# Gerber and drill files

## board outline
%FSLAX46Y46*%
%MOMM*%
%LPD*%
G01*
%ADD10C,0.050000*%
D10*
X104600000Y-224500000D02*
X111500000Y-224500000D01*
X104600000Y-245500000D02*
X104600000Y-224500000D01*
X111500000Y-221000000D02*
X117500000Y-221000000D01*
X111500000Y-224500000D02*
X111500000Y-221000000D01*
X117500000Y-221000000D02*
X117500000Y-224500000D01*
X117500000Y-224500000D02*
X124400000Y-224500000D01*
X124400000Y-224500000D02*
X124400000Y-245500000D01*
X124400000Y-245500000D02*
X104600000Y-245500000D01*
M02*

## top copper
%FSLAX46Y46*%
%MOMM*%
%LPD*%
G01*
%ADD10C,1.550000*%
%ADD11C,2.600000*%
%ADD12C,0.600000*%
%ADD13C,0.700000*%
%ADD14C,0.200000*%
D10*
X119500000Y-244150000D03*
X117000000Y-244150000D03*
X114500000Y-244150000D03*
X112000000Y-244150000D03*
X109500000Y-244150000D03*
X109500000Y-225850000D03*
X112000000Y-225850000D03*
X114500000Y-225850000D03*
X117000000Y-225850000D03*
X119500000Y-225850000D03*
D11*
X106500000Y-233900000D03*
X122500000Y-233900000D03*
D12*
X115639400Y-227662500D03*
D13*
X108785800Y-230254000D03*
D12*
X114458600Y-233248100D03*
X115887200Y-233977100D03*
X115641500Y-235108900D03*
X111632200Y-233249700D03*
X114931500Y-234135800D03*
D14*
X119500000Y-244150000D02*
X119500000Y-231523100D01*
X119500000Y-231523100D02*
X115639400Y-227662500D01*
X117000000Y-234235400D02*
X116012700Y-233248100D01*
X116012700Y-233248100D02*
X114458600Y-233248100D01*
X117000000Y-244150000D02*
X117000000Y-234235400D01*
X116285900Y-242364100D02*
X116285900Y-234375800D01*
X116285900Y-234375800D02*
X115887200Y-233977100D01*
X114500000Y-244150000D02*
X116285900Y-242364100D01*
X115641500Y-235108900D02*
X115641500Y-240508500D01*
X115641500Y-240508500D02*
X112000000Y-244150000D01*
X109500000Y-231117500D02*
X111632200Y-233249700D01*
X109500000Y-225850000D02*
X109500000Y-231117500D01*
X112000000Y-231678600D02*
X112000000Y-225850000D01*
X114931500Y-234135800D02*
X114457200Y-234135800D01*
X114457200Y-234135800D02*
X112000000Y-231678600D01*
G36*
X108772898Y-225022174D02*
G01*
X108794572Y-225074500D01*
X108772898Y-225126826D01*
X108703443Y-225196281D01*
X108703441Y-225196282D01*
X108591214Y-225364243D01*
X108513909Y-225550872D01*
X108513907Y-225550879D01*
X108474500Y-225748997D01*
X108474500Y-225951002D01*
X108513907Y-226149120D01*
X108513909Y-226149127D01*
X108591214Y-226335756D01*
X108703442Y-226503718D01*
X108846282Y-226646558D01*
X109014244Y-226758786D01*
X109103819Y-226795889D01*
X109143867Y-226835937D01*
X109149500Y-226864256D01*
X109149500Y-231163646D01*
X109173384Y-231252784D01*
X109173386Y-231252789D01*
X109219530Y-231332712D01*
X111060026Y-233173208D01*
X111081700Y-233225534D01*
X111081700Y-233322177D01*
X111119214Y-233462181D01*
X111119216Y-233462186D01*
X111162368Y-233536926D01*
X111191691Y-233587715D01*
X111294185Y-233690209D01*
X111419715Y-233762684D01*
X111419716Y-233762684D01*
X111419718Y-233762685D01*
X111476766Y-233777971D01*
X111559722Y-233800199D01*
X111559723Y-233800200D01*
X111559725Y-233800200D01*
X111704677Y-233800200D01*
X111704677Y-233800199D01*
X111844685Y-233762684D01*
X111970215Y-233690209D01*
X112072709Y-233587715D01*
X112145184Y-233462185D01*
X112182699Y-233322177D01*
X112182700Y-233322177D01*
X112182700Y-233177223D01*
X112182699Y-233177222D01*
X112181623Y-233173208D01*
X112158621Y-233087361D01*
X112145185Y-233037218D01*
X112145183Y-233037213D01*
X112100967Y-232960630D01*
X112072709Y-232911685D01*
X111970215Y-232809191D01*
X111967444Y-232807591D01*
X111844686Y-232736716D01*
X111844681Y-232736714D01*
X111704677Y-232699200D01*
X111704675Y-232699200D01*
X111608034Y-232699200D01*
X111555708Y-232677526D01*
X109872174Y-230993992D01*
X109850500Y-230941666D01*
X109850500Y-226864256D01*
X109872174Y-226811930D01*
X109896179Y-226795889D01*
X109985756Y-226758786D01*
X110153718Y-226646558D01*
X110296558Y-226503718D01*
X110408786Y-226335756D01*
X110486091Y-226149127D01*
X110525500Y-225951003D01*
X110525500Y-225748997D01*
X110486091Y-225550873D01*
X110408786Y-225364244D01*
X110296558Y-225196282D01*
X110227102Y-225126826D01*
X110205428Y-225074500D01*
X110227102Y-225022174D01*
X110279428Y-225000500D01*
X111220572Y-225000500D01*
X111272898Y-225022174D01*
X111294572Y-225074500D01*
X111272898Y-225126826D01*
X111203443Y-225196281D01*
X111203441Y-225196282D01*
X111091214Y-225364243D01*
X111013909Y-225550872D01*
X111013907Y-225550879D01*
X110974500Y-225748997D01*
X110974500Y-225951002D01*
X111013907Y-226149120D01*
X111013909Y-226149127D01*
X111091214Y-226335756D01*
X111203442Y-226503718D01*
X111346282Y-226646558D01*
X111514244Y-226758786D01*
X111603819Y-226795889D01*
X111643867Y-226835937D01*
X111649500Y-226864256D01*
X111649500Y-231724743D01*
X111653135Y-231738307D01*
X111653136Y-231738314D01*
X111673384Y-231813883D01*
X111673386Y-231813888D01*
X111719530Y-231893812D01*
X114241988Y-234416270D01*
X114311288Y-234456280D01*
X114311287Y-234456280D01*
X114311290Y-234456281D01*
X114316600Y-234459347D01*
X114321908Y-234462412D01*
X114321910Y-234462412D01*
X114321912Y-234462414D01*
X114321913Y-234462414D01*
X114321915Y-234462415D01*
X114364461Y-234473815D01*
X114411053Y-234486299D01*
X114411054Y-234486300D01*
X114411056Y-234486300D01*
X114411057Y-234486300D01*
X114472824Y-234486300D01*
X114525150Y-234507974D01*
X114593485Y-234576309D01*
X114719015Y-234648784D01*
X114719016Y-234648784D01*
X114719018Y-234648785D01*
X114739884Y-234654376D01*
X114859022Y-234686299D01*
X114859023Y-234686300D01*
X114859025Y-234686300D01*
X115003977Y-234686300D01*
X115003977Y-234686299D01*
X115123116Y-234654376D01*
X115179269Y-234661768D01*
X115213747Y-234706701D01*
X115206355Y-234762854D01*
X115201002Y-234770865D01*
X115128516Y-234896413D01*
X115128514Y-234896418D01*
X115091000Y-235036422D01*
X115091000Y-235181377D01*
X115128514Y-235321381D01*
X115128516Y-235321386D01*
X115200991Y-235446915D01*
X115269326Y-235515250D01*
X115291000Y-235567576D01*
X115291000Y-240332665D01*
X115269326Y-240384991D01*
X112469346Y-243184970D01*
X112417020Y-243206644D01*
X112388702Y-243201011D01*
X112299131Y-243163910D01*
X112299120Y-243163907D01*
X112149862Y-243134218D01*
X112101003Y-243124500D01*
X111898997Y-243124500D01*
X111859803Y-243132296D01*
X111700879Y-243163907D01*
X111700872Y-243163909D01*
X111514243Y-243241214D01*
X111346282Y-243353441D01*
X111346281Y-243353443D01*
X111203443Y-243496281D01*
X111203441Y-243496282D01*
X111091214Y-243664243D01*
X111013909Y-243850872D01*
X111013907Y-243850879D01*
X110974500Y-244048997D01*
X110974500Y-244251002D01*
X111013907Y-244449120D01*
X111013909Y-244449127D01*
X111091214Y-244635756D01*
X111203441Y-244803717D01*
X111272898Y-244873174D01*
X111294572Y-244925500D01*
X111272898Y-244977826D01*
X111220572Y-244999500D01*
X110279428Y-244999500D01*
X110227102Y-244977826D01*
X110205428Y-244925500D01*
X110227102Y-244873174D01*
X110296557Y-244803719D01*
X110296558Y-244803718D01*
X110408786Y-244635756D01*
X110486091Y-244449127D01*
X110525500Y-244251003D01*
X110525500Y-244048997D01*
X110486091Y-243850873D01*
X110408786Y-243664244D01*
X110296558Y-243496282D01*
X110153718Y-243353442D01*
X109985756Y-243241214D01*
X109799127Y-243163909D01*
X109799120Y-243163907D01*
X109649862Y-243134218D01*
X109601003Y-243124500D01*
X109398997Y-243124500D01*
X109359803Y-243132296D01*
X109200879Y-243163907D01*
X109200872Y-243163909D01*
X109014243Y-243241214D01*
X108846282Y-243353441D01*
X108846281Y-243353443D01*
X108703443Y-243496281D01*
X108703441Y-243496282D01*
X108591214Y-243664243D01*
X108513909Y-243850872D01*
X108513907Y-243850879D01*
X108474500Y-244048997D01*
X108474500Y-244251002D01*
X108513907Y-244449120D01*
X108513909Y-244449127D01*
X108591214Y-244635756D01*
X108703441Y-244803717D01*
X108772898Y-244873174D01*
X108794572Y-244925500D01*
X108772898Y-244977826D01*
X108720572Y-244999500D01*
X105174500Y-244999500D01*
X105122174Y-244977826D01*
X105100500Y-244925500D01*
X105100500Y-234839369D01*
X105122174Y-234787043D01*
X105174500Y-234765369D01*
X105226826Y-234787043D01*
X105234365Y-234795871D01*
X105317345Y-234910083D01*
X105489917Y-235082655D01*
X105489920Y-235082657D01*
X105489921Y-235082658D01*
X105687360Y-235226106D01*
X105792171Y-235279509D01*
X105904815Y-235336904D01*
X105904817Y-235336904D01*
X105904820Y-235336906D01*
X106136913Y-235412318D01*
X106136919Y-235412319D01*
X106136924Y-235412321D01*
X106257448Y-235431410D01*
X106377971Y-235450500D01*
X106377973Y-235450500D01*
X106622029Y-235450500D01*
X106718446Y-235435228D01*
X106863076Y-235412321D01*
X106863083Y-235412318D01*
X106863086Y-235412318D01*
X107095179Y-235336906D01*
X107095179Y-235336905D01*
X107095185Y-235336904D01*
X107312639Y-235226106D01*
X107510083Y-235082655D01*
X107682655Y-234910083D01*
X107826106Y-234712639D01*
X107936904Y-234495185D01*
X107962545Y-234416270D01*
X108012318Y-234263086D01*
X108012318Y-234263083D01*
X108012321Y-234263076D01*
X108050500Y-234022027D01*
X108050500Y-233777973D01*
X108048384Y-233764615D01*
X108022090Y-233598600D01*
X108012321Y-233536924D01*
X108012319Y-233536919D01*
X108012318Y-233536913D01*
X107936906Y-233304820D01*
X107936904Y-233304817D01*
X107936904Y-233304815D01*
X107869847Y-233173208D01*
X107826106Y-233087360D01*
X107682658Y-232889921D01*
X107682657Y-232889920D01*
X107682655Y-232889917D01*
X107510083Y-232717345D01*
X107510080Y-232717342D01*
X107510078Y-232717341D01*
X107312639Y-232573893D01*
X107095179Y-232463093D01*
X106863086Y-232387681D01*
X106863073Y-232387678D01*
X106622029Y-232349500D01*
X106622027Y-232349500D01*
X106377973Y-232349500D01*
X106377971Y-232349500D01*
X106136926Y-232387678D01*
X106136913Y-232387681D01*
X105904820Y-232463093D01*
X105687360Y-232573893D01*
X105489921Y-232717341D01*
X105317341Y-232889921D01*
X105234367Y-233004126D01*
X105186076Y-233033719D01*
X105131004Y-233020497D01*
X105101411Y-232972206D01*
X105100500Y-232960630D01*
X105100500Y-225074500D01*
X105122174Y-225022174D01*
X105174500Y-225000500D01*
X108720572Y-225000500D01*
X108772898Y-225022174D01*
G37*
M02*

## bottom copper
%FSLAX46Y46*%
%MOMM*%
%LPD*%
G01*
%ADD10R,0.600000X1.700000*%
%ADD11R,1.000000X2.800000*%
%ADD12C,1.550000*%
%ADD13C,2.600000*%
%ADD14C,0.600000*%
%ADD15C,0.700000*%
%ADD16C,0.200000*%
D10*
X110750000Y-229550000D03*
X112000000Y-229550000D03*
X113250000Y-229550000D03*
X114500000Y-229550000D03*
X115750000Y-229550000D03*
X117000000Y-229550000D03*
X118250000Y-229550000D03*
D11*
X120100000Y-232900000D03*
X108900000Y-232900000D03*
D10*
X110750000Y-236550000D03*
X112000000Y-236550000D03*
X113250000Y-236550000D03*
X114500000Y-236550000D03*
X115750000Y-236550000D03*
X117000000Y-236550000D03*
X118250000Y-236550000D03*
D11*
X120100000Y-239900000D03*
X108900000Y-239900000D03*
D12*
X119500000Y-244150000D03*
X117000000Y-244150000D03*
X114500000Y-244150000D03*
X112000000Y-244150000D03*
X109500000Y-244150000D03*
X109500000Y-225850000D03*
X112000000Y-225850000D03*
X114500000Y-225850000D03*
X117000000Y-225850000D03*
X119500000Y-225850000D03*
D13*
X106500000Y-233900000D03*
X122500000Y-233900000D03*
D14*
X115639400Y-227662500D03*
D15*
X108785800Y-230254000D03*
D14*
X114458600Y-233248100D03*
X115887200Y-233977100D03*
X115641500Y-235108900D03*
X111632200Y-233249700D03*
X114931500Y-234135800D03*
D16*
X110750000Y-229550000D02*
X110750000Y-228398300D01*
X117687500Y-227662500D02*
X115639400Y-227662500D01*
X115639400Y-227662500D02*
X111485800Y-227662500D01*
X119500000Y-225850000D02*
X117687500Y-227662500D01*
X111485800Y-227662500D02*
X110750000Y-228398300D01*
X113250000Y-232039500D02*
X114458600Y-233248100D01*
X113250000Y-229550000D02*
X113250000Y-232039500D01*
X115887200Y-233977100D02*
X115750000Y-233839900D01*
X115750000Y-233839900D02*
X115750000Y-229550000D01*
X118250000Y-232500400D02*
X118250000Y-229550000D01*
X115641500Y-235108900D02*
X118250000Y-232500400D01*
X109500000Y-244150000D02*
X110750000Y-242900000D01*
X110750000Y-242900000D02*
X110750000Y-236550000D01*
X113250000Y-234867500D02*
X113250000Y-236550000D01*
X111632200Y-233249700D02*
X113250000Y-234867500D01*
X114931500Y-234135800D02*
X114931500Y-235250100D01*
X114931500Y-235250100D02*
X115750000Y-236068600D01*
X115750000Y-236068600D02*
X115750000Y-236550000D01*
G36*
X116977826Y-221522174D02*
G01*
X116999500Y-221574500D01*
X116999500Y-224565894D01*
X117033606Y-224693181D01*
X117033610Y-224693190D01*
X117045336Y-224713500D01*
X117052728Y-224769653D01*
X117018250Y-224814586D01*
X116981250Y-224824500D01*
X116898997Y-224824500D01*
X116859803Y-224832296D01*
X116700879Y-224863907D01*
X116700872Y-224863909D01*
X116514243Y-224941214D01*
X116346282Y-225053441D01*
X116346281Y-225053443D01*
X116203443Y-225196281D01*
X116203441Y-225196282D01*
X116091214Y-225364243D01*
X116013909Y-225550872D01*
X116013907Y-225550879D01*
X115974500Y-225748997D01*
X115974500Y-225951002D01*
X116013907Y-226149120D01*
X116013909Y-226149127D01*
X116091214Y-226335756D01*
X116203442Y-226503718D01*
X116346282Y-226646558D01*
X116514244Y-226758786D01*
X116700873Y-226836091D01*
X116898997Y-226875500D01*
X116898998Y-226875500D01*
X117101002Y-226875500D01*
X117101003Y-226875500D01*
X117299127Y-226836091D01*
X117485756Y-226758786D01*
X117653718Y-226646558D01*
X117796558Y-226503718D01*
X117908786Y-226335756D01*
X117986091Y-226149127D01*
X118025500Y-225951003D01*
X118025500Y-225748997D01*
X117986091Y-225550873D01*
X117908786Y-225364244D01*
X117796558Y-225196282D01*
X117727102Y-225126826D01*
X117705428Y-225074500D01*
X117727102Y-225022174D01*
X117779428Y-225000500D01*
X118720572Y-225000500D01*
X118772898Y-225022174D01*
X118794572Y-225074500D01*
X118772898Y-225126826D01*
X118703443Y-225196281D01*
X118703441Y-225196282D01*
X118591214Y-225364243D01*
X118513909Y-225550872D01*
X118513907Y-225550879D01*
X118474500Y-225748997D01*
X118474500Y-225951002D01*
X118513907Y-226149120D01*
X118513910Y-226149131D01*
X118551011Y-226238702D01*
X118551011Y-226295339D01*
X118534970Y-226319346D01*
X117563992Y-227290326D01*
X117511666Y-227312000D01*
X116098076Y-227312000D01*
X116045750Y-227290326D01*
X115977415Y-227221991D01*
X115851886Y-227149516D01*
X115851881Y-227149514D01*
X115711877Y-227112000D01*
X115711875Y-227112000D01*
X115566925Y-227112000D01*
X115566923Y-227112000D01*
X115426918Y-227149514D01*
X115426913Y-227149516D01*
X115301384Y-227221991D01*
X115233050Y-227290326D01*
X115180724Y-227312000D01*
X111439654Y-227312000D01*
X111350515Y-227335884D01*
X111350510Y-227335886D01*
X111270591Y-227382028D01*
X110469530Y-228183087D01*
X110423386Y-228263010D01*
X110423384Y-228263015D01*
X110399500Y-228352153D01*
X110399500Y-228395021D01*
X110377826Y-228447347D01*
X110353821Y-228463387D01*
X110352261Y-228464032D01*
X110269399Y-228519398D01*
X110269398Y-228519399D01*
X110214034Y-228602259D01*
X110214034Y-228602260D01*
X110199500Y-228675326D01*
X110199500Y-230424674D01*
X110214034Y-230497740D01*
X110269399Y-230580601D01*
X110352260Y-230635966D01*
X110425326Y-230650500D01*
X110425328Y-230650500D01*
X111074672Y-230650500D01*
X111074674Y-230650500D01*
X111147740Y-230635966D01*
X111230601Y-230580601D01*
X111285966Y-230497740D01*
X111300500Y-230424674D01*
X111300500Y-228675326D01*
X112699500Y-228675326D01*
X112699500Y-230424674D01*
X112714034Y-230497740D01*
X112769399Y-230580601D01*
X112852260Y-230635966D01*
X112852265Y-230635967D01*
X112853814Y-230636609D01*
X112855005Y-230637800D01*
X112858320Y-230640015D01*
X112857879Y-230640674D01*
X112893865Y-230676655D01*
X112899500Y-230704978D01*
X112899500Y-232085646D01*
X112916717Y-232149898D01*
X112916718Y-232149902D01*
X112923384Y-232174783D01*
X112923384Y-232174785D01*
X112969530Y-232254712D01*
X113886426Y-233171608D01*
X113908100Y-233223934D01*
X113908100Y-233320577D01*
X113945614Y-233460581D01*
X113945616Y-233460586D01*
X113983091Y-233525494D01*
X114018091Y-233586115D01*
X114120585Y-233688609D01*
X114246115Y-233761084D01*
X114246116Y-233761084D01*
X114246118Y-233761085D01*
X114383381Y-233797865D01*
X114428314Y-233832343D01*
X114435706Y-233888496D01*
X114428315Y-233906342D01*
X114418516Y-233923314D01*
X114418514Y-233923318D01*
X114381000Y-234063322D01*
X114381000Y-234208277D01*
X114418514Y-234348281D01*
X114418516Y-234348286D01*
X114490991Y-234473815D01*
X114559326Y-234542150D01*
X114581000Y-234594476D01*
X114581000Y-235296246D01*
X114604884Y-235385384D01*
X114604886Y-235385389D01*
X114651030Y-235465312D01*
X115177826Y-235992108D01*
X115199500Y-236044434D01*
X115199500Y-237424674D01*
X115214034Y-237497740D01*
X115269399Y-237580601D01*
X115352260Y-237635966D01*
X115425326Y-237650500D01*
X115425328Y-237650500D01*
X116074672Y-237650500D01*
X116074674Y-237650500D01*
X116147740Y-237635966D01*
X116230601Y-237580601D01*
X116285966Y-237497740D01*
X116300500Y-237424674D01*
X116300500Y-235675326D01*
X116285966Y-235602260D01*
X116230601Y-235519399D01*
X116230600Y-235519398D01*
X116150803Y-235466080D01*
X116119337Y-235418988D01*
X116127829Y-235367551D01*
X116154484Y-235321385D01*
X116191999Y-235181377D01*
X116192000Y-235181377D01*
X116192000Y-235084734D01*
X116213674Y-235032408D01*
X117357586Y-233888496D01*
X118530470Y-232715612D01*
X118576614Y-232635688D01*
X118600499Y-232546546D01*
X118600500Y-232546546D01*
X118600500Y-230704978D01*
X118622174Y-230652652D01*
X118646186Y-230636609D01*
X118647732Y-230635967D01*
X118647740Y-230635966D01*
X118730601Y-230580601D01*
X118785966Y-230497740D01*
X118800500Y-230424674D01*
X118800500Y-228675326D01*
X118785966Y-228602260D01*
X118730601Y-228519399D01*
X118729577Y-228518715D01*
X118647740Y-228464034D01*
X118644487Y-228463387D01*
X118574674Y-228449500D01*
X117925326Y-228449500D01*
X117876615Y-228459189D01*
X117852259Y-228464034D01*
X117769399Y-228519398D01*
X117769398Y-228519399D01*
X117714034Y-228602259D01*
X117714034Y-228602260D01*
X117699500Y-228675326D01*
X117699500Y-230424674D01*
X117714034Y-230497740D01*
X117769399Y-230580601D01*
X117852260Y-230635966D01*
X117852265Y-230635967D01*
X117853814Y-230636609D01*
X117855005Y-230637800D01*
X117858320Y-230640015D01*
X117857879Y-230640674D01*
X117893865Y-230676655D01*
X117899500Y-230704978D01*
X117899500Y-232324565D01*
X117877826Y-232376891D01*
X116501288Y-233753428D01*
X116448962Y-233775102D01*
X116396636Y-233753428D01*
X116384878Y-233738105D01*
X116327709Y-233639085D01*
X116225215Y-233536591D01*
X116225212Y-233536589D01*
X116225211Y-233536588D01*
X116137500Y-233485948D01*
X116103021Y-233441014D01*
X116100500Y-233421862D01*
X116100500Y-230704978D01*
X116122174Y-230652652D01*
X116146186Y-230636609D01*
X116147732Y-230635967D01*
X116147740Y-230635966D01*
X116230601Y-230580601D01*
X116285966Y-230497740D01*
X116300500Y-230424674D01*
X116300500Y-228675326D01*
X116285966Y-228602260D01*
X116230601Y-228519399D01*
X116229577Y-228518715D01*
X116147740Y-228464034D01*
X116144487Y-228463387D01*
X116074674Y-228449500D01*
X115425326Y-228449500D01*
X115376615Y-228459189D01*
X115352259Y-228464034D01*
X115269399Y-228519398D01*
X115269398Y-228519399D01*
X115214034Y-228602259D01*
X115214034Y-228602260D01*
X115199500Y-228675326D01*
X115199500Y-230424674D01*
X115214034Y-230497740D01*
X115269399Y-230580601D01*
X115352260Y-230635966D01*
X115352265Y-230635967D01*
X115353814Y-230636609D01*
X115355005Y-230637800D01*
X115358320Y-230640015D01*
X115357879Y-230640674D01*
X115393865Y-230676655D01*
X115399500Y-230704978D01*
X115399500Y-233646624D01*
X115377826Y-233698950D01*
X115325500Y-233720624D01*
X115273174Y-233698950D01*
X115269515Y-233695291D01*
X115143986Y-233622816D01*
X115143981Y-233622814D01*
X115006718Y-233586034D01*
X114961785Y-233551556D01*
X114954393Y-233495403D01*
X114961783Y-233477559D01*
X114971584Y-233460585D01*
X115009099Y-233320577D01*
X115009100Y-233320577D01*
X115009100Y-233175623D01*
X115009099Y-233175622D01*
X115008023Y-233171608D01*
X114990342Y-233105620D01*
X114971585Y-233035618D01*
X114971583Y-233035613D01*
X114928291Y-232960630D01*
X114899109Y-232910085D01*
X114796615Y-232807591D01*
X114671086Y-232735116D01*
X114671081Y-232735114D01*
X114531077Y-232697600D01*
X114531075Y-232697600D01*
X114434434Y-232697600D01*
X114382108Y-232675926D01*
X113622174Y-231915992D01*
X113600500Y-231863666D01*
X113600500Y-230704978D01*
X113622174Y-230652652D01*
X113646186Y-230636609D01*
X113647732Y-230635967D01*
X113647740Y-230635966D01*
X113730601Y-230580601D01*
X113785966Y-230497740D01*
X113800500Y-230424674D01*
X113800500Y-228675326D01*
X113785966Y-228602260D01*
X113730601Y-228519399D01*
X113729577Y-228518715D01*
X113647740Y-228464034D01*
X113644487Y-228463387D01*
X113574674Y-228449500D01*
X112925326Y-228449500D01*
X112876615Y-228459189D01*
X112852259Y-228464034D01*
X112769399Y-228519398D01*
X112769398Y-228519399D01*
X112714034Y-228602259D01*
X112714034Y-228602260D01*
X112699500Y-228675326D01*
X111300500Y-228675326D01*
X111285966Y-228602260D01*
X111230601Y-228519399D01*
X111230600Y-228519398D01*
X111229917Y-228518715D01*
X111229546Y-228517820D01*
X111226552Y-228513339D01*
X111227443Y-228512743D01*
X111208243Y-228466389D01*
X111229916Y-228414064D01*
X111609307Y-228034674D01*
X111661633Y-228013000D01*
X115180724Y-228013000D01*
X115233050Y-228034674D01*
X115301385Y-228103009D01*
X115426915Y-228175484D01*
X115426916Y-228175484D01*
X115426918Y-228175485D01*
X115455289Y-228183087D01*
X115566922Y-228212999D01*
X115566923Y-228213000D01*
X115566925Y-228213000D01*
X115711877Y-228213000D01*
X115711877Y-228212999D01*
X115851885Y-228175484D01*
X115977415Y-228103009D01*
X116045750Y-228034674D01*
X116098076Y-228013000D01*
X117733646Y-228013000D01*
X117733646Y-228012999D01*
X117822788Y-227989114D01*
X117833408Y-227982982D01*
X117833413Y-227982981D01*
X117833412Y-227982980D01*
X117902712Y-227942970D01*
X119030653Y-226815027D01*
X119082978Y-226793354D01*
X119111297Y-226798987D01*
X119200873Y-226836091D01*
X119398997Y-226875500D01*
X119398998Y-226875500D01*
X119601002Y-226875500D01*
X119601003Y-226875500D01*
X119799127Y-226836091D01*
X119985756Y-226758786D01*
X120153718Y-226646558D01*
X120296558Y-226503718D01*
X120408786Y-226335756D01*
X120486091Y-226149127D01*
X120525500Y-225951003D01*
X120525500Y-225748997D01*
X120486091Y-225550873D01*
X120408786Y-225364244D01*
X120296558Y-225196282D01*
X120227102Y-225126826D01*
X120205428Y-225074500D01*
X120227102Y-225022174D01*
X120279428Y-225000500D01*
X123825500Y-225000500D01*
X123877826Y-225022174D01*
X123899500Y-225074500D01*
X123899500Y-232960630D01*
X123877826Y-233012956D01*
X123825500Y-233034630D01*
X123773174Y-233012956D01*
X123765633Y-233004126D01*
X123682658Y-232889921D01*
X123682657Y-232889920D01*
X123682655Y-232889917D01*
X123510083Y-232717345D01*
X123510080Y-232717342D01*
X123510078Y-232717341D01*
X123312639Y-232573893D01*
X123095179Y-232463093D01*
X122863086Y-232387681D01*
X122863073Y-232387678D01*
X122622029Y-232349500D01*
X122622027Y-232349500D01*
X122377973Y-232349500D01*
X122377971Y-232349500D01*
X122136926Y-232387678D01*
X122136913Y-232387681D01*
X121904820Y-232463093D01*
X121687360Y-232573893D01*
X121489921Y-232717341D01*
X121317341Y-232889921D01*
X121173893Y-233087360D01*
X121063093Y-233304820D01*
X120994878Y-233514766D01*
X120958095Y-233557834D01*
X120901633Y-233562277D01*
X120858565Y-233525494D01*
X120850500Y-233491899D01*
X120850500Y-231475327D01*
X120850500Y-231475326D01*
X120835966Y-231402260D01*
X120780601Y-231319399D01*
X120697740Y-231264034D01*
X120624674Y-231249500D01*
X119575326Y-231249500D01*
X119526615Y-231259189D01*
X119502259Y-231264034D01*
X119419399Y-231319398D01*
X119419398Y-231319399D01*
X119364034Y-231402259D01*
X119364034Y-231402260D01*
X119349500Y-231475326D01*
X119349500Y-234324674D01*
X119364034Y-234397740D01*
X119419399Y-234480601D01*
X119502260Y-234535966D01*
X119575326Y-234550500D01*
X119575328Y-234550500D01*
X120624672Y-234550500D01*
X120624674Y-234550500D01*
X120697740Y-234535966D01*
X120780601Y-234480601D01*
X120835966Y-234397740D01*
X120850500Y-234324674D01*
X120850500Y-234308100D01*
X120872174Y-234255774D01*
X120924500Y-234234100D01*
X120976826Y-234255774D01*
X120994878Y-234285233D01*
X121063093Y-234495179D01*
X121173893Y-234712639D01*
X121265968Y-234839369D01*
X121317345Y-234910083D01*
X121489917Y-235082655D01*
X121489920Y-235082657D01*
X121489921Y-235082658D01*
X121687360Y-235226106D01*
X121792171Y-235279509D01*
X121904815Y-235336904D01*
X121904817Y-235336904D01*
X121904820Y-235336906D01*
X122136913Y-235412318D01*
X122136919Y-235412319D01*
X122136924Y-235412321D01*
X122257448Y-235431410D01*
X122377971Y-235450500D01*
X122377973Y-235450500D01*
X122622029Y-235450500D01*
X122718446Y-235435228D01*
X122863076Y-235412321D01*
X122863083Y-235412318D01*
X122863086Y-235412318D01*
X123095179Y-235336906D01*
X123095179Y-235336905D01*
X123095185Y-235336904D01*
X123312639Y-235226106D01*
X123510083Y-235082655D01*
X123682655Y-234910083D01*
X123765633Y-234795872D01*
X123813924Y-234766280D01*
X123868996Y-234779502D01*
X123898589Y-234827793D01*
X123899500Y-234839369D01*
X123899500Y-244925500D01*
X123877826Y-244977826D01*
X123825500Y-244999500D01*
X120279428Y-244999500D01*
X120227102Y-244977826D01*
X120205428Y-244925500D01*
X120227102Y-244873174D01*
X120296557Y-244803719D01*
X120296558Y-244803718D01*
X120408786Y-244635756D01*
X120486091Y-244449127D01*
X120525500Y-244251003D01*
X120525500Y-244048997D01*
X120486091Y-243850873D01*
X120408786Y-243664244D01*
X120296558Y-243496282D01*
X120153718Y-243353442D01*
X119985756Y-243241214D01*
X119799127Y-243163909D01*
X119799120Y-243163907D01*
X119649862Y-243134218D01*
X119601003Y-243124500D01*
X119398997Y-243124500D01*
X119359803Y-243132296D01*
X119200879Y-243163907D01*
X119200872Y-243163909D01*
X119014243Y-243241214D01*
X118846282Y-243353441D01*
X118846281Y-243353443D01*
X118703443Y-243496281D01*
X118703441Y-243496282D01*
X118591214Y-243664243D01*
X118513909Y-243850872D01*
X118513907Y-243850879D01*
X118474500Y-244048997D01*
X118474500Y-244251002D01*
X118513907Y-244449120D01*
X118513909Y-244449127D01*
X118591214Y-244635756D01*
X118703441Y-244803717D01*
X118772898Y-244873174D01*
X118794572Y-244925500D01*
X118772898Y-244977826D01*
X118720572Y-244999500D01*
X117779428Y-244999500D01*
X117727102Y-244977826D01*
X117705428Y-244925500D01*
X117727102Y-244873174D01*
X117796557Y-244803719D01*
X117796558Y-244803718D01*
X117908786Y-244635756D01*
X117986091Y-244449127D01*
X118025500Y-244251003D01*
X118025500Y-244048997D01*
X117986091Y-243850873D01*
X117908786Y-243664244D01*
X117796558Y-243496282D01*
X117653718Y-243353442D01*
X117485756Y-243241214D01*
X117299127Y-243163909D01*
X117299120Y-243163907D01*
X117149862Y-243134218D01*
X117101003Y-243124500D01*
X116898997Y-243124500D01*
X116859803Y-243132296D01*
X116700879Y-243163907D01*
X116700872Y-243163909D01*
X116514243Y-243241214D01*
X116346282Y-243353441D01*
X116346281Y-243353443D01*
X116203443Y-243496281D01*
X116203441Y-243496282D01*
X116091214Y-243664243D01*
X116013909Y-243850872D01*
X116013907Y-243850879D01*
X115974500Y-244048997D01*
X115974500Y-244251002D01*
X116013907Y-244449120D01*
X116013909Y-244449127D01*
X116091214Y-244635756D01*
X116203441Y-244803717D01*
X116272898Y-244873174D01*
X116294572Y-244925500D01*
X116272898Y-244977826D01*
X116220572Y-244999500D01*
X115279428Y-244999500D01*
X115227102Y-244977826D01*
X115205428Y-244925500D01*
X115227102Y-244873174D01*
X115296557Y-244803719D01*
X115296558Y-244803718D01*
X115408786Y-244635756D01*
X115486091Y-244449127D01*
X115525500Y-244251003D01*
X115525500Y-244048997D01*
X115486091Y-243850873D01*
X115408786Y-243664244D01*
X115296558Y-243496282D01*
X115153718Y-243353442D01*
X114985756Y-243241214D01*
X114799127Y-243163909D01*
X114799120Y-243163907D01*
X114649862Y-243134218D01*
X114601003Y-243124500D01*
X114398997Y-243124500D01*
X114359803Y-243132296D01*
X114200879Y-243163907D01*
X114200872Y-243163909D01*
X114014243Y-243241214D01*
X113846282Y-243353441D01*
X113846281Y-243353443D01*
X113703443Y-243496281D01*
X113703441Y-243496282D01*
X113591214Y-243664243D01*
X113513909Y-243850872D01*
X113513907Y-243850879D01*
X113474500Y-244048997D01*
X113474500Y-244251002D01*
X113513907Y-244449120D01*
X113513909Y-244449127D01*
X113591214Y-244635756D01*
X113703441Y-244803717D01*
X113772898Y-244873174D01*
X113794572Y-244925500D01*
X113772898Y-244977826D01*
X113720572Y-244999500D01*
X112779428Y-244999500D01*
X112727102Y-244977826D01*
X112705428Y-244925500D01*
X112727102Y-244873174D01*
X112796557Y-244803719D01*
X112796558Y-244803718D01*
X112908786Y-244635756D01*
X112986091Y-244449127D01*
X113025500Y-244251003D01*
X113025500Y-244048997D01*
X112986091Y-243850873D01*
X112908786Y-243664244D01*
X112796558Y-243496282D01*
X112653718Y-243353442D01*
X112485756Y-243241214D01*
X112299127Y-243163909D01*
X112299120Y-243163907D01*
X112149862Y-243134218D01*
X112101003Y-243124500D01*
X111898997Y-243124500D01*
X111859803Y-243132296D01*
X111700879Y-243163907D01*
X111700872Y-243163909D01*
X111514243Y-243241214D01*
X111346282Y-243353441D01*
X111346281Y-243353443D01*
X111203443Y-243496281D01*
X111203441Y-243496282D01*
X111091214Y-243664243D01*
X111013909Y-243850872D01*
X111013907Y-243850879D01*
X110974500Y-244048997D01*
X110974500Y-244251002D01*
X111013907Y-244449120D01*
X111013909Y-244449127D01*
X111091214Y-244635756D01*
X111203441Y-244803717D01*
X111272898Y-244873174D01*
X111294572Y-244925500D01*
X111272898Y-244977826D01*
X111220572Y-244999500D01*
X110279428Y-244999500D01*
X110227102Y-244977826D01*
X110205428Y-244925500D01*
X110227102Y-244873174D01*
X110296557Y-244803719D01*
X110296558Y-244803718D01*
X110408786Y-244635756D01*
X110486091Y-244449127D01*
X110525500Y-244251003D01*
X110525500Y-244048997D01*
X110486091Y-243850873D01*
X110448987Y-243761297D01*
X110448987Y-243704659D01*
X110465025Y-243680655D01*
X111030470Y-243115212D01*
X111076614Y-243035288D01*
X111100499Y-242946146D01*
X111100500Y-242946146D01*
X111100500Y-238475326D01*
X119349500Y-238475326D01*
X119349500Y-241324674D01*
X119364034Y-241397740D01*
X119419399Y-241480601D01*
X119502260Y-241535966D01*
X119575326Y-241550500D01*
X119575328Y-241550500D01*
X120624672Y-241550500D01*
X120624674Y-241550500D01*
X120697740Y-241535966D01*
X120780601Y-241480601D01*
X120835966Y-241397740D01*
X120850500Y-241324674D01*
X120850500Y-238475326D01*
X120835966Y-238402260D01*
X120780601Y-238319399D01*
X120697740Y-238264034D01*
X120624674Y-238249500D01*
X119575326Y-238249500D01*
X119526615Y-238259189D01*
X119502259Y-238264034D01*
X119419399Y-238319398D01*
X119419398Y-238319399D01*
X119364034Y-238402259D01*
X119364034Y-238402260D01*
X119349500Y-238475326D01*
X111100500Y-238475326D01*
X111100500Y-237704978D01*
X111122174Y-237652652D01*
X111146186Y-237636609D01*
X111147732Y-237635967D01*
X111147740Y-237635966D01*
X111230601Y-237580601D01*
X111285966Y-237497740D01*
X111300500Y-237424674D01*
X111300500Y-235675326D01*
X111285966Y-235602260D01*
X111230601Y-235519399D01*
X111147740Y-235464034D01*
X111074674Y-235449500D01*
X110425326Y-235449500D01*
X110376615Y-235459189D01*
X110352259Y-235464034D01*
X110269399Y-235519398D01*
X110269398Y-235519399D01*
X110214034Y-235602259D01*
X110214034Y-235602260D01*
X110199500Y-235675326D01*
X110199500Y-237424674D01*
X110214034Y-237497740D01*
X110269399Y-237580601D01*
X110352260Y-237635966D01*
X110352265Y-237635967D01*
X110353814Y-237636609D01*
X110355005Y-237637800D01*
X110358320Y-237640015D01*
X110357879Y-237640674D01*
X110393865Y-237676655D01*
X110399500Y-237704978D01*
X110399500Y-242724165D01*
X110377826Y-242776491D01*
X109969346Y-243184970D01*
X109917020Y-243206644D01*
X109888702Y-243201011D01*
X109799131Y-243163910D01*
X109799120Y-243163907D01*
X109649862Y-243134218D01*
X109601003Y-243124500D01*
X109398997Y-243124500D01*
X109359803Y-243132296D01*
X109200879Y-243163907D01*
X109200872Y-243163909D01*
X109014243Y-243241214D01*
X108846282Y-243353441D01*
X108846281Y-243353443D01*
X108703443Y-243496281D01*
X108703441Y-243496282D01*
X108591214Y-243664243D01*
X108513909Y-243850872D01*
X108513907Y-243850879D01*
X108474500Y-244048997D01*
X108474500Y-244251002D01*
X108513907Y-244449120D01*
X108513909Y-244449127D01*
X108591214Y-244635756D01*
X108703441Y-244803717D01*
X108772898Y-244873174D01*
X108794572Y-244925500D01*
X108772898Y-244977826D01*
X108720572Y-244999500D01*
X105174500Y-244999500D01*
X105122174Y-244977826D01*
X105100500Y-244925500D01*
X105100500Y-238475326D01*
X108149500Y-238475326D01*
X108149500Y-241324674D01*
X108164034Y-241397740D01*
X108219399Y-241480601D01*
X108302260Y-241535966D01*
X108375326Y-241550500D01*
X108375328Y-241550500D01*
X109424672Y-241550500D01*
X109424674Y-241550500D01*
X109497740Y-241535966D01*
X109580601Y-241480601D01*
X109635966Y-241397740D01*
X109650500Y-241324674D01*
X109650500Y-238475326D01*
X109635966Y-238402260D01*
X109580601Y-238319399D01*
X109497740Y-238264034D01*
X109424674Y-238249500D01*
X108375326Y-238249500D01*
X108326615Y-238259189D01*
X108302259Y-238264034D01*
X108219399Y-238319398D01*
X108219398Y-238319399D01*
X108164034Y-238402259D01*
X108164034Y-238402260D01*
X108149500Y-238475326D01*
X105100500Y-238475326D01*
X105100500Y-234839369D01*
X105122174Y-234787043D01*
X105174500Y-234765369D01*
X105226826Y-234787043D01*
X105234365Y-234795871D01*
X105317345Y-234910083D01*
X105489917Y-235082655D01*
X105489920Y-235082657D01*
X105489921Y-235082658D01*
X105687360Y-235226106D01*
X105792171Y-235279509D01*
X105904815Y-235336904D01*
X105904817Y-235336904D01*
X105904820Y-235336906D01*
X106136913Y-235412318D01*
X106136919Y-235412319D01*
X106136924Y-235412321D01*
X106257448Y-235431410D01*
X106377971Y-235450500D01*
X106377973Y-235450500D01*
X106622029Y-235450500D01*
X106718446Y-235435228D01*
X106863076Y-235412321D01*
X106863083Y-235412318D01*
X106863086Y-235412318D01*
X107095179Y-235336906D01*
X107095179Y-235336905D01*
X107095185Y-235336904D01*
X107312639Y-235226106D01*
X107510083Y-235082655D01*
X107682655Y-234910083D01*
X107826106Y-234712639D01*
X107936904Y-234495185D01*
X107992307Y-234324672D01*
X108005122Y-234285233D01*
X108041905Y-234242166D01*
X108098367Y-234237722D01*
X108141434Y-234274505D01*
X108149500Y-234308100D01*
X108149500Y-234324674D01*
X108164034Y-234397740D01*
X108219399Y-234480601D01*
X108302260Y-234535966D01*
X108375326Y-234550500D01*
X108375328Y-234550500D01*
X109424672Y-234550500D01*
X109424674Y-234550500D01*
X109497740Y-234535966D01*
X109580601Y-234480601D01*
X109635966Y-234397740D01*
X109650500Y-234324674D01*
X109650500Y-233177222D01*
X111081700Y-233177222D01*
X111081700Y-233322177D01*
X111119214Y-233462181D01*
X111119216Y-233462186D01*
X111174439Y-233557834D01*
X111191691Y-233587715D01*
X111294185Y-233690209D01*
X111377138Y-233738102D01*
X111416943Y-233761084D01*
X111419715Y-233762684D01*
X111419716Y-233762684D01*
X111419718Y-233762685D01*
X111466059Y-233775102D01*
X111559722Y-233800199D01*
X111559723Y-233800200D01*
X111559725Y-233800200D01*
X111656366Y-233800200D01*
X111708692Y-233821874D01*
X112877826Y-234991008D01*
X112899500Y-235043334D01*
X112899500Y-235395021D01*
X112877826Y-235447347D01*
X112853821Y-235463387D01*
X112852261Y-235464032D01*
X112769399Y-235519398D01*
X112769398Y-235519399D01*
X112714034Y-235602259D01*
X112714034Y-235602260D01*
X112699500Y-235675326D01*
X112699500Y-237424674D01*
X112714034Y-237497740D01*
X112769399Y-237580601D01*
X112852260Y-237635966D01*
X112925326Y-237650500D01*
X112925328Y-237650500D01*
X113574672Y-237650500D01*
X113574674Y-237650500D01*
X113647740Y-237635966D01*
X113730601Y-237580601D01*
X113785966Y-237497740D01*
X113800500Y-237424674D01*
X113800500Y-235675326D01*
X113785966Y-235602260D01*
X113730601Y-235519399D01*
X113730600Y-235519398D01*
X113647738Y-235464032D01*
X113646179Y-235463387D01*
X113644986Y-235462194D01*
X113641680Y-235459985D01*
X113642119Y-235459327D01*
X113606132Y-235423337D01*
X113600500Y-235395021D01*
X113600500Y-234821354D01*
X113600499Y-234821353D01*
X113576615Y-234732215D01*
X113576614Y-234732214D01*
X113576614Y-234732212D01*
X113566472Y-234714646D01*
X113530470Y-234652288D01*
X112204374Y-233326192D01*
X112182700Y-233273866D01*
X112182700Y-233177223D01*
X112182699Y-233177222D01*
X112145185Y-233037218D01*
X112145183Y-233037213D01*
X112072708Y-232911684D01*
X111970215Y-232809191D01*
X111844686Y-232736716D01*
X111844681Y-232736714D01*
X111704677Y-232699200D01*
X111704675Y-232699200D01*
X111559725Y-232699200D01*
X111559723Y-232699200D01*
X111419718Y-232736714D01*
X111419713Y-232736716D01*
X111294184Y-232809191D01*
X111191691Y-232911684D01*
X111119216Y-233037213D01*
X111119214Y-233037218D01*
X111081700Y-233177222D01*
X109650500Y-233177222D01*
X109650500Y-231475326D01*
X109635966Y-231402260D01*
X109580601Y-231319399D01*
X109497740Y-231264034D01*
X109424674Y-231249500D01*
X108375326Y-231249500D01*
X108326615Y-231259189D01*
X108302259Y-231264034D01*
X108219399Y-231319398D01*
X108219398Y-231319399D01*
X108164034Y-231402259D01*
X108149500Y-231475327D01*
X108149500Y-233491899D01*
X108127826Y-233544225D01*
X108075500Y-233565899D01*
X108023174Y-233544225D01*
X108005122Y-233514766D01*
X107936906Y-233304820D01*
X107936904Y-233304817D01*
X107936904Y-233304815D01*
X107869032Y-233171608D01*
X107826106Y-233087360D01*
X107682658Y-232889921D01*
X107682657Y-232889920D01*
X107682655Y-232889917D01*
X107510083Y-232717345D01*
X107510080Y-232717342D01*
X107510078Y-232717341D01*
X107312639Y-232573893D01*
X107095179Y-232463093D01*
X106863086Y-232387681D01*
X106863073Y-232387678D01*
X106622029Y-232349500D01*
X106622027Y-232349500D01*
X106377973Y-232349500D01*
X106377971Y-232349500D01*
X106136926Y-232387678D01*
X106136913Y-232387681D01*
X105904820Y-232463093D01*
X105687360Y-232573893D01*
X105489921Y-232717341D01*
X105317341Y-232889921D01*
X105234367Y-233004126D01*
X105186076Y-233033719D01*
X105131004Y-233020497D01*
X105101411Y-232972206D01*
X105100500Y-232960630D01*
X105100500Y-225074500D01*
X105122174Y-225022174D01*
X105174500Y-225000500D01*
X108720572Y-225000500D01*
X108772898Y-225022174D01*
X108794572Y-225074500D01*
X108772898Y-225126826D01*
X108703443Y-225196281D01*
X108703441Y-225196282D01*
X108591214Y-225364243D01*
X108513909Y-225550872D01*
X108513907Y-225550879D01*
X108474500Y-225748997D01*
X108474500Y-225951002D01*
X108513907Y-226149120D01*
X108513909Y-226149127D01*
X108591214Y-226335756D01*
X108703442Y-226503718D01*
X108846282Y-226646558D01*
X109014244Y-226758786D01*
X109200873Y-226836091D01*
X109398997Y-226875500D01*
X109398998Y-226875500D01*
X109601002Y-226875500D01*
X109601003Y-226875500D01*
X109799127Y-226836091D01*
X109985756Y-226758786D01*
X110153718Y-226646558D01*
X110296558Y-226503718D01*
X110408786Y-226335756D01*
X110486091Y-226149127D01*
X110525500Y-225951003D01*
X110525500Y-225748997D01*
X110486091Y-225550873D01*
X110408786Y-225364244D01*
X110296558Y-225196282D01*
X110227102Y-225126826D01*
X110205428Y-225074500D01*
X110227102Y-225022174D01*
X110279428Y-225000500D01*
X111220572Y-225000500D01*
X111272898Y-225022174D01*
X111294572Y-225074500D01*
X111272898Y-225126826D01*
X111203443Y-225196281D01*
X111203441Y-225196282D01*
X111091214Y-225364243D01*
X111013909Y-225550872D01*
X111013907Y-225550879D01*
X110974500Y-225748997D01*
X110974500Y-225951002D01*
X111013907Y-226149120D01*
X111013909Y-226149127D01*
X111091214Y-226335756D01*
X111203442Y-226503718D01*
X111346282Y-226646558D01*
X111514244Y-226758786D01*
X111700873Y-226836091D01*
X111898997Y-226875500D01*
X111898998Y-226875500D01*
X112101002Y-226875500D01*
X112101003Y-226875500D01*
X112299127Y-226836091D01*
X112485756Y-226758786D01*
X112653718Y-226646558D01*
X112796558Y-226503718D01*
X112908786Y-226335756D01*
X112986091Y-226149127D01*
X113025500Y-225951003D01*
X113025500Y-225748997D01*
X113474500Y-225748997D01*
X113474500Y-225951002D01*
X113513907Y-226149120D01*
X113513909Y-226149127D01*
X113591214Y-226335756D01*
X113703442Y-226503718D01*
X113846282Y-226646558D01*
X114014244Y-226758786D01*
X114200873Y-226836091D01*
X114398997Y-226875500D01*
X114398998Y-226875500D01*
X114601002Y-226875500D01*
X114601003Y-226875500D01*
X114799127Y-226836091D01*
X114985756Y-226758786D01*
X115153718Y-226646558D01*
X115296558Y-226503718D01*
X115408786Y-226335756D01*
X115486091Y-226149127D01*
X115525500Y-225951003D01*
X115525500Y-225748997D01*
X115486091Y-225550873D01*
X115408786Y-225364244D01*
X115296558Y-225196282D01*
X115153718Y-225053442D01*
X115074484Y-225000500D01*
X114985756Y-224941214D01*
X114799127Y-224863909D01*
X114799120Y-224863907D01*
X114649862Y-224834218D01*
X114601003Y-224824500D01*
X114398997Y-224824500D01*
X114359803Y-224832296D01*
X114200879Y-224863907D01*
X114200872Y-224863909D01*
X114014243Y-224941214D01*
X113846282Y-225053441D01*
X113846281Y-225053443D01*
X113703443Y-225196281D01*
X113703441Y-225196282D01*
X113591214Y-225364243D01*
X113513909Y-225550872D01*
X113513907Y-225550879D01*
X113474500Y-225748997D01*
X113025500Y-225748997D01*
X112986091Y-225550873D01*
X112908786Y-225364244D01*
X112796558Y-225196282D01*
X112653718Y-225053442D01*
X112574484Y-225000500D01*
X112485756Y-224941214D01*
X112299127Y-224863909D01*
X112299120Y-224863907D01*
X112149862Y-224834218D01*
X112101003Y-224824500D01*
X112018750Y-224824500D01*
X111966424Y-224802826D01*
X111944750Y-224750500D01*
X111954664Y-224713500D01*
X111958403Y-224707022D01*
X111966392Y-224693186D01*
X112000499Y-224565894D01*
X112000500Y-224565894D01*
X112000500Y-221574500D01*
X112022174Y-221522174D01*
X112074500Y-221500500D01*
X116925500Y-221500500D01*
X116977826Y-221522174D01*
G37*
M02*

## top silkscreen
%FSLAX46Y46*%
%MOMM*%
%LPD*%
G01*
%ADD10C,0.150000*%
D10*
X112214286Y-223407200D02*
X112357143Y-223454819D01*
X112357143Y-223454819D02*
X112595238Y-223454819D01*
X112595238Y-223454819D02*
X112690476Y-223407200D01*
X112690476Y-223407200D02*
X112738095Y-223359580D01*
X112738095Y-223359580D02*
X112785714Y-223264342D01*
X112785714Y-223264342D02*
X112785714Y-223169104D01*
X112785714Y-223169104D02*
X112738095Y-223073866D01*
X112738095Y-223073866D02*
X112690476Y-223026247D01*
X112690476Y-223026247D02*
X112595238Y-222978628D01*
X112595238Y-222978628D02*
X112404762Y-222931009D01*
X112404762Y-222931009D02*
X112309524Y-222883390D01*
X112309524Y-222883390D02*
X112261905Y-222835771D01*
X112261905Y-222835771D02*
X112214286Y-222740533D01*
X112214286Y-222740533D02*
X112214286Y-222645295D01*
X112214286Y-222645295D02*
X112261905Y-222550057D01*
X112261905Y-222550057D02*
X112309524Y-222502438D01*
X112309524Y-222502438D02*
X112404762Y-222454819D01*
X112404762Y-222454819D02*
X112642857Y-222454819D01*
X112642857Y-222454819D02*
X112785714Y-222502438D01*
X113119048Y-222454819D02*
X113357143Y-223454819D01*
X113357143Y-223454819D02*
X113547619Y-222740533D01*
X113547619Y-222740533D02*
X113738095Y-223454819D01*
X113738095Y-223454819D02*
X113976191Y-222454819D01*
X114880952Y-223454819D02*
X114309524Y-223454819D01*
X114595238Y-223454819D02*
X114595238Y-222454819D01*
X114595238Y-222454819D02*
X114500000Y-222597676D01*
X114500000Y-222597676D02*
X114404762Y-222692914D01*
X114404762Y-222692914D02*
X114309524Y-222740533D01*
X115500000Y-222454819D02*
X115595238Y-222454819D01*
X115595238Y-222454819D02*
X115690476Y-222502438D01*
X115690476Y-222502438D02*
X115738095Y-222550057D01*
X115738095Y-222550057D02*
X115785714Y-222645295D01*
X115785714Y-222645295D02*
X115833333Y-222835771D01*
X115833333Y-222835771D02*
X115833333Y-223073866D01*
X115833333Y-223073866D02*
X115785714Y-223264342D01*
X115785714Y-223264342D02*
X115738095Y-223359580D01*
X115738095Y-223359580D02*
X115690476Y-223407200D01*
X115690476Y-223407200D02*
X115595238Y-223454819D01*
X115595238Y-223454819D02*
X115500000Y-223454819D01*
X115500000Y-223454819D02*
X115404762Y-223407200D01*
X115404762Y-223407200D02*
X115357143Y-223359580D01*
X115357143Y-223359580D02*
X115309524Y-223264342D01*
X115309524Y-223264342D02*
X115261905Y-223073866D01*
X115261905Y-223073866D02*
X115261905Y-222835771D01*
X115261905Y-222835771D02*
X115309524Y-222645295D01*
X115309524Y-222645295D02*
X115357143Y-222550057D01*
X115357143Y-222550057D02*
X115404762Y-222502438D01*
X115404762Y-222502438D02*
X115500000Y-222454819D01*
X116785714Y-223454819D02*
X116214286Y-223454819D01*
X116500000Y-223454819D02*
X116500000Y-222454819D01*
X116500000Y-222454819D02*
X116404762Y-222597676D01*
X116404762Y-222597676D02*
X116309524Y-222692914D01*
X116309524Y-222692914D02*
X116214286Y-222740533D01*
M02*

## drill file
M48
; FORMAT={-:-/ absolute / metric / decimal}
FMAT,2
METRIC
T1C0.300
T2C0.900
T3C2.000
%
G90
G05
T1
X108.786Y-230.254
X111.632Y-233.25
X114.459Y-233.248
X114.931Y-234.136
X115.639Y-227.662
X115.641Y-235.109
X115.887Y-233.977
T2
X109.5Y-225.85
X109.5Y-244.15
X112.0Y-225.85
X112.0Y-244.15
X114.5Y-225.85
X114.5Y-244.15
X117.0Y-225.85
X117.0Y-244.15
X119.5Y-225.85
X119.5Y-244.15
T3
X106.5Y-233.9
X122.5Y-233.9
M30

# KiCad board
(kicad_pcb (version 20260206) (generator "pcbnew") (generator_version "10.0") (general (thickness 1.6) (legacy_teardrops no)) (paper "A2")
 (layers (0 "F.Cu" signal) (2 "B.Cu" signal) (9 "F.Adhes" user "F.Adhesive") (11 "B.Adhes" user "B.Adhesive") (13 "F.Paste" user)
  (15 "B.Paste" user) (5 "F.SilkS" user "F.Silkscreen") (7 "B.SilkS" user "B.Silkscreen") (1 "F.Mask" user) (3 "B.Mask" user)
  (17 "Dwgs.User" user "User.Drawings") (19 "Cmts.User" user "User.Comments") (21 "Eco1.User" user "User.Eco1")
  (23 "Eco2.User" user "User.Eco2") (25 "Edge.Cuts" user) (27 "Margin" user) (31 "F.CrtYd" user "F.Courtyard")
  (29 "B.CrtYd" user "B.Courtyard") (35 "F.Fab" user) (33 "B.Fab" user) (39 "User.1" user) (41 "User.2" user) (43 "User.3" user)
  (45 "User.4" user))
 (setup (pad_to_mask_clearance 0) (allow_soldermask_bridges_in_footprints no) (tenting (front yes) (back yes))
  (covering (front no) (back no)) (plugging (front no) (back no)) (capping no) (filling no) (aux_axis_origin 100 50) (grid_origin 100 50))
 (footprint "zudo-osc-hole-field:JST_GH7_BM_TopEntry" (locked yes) (layer "B.Cu") (at 114.5 229.55 180)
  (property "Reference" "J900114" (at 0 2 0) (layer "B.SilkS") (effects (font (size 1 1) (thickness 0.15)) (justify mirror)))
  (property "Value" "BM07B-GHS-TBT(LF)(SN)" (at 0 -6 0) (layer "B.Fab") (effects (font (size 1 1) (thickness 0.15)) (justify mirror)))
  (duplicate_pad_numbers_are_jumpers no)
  (pad "1" smd rect (at 3.75 0 180) (size 0.6 1.7) (layers "B.Cu" "B.Mask" "B.Paste") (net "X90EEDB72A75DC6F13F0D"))
  (pad "2" smd rect (at 2.5 0 180) (size 0.6 1.7) (layers "B.Cu" "B.Mask" "B.Paste") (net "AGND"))
  (pad "3" smd rect (at 1.25 0 180) (size 0.6 1.7) (layers "B.Cu" "B.Mask" "B.Paste") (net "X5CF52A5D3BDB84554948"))
  (pad "4" smd rect (at 0 0 180) (size 0.6 1.7) (layers "B.Cu" "B.Mask" "B.Paste") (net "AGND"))
  (pad "5" smd rect (at -1.25 0 180) (size 0.6 1.7) (layers "B.Cu" "B.Mask" "B.Paste") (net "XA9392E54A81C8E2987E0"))
  (pad "6" smd rect (at -2.5 0 180) (size 0.6 1.7) (layers "B.Cu" "B.Mask" "B.Paste") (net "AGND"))
  (pad "7" smd rect (at -3.75 0 180) (size 0.6 1.7) (layers "B.Cu" "B.Mask" "B.Paste") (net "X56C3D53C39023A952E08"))
  (pad "MP1" smd rect (at -5.6 -3.35 180) (size 1 2.8) (layers "B.Cu" "B.Mask" "B.Paste") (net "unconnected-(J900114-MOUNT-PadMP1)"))
  (pad "MP2" smd rect (at 5.6 -3.35 180) (size 1 2.8) (layers "B.Cu" "B.Mask" "B.Paste") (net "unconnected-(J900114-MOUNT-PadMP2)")))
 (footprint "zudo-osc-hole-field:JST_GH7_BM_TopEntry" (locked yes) (layer "B.Cu") (at 114.5 236.55 180)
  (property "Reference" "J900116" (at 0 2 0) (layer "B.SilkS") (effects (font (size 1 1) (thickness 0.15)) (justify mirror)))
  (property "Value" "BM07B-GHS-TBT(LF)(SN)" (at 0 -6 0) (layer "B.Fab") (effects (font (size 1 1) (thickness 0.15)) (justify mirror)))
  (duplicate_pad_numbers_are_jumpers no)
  (pad "1" smd rect (at 3.75 0 180) (size 0.6 1.7) (layers "B.Cu" "B.Mask" "B.Paste") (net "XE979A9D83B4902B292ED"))
  (pad "2" smd rect (at 2.5 0 180) (size 0.6 1.7) (layers "B.Cu" "B.Mask" "B.Paste") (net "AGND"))
  (pad "3" smd rect (at 1.25 0 180) (size 0.6 1.7) (layers "B.Cu" "B.Mask" "B.Paste") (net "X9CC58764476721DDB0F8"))
  (pad "4" smd rect (at 0 0 180) (size 0.6 1.7) (layers "B.Cu" "B.Mask" "B.Paste") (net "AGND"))
  (pad "5" smd rect (at -1.25 0 180) (size 0.6 1.7) (layers "B.Cu" "B.Mask" "B.Paste") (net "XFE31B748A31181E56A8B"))
  (pad "6" smd rect (at -2.5 0 180) (size 0.6 1.7) (layers "B.Cu" "B.Mask" "B.Paste") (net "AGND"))
  (pad "7" smd rect (at -3.75 0 180) (size 0.6 1.7) (layers "B.Cu" "B.Mask" "B.Paste") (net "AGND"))
  (pad "MP1" smd rect (at -5.6 -3.35 180) (size 1 2.8) (layers "B.Cu" "B.Mask" "B.Paste") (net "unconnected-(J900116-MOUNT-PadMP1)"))
  (pad "MP2" smd rect (at 5.6 -3.35 180) (size 1 2.8) (layers "B.Cu" "B.Mask" "B.Paste") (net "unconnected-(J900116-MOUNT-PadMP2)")))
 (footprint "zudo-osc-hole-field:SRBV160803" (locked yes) (layer "F.Cu") (at 114.5 235)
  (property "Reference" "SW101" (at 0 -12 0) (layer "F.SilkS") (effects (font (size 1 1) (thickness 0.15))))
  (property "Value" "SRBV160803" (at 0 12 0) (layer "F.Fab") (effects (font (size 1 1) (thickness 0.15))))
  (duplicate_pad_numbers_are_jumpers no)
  (pad "1" thru_hole circle (at 5 9.15) (size 1.55 1.55) (drill 0.9) (layers "*.Cu" "*.Mask") (remove_unused_layers no)
   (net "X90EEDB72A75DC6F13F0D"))
  (pad "2" thru_hole circle (at 2.5 9.15) (size 1.55 1.55) (drill 0.9) (layers "*.Cu" "*.Mask") (remove_unused_layers no)
   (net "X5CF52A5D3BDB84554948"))
  (pad "3" thru_hole circle (at 0 9.15) (size 1.55 1.55) (drill 0.9) (layers "*.Cu" "*.Mask") (remove_unused_layers no)
   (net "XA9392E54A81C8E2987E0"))
  (pad "4" thru_hole circle (at -2.5 9.15) (size 1.55 1.55) (drill 0.9) (layers "*.Cu" "*.Mask") (remove_unused_layers no)
   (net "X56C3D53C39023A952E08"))
  (pad "5" thru_hole circle (at -5 9.15) (size 1.55 1.55) (drill 0.9) (layers "*.Cu" "*.Mask") (remove_unused_layers no)
   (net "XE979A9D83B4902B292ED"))
  (pad "6" thru_hole circle (at -5 -9.15) (size 1.55 1.55) (drill 0.9) (layers "*.Cu" "*.Mask") (remove_unused_layers no)
   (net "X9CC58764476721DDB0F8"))
  (pad "7" thru_hole circle (at -2.5 -9.15) (size 1.55 1.55) (drill 0.9) (layers "*.Cu" "*.Mask") (remove_unused_layers no)
   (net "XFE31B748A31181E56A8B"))
  (pad "8" thru_hole circle (at 0 -9.15) (size 1.55 1.55) (drill 0.9) (layers "*.Cu" "*.Mask") (remove_unused_layers no)
   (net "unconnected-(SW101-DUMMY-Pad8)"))
  (pad "9" thru_hole circle (at 2.5 -9.15) (size 1.55 1.55) (drill 0.9) (layers "*.Cu" "*.Mask") (remove_unused_layers no)
   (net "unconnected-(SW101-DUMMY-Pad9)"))
  (pad "10" thru_hole circle (at 5 -9.15) (size 1.55 1.55) (drill 0.9) (layers "*.Cu" "*.Mask") (remove_unused_layers no)
   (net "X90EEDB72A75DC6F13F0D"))
  (pad "MP1" thru_hole circle (at -8 -1.1) (size 2.6 2.6) (drill 2) (layers "*.Cu" "*.Mask") (remove_unused_layers no)
   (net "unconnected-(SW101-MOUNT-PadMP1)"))
  (pad "MP2" thru_hole circle (at 8 -1.1) (size 2.6 2.6) (drill 2) (layers "*.Cu" "*.Mask") (remove_unused_layers no)
   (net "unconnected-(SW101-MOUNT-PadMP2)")))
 (gr_line (start 104.6 224.5) (end 111.5 224.5) (stroke (width 0.05) (type default)) (layer "Edge.Cuts"))
 (gr_line (start 104.6 245.5) (end 104.6 224.5) (stroke (width 0.05) (type default)) (layer "Edge.Cuts"))
 (gr_line (start 111.5 221) (end 117.5 221) (stroke (width 0.05) (type default)) (layer "Edge.Cuts"))
 (gr_line (start 111.5 224.5) (end 111.5 221) (stroke (width 0.05) (type default)) (layer "Edge.Cuts"))
 (gr_line (start 117.5 221) (end 117.5 224.5) (stroke (width 0.05) (type default)) (layer "Edge.Cuts"))
 (gr_line (start 117.5 224.5) (end 124.4 224.5) (stroke (width 0.05) (type default)) (layer "Edge.Cuts"))
 (gr_line (start 124.4 224.5) (end 124.4 245.5) (stroke (width 0.05) (type default)) (layer "Edge.Cuts"))
 (gr_line (start 124.4 245.5) (end 104.6 245.5) (stroke (width 0.05) (type default)) (layer "Edge.Cuts"))
 (segment (start 119.5 244.15) (end 119.5 231.5231) (width 0.2) (layer "F.Cu") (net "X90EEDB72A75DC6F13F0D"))
 (segment (start 119.5 231.5231) (end 115.6394 227.6625) (width 0.2) (layer "F.Cu") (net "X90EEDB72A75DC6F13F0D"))
 (via (at 115.6394 227.6625) (size 0.6) (drill 0.3) (layers "F.Cu" "B.Cu") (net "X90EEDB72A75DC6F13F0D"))
 (segment (start 110.75 229.55) (end 110.75 228.3983) (width 0.2) (layer "B.Cu") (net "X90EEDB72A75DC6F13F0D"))
 (segment (start 117.6875 227.6625) (end 115.6394 227.6625) (width 0.2) (layer "B.Cu") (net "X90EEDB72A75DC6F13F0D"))
 (segment (start 115.6394 227.6625) (end 111.4858 227.6625) (width 0.2) (layer "B.Cu") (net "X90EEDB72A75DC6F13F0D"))
 (segment (start 119.5 225.85) (end 117.6875 227.6625) (width 0.2) (layer "B.Cu") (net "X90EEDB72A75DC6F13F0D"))
 (segment (start 111.4858 227.6625) (end 110.75 228.3983) (width 0.2) (layer "B.Cu") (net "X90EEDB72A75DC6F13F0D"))
 (via (at 108.7858 230.254) (size 0.7) (drill 0.3) (layers "F.Cu" "B.Cu") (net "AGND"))
 (segment (start 117 234.2354) (end 116.0127 233.2481) (width 0.2) (layer "F.Cu") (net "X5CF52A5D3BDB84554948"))
 (segment (start 116.0127 233.2481) (end 114.4586 233.2481) (width 0.2) (layer "F.Cu") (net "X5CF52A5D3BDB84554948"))
 (segment (start 117 244.15) (end 117 234.2354) (width 0.2) (layer "F.Cu") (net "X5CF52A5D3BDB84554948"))
 (via (at 114.4586 233.2481) (size 0.6) (drill 0.3) (layers "F.Cu" "B.Cu") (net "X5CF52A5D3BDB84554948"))
 (segment (start 113.25 232.0395) (end 114.4586 233.2481) (width 0.2) (layer "B.Cu") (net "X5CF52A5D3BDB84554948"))
 (segment (start 113.25 229.55) (end 113.25 232.0395) (width 0.2) (layer "B.Cu") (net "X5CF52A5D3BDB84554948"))
 (segment (start 116.2859 242.3641) (end 116.2859 234.3758) (width 0.2) (layer "F.Cu") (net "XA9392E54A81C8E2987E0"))
 (segment (start 116.2859 234.3758) (end 115.8872 233.9771) (width 0.2) (layer "F.Cu") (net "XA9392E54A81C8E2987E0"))
 (segment (start 114.5 244.15) (end 116.2859 242.3641) (width 0.2) (layer "F.Cu") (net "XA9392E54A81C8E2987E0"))
 (via (at 115.8872 233.9771) (size 0.6) (drill 0.3) (layers "F.Cu" "B.Cu") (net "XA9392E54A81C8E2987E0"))
 (segment (start 115.8872 233.9771) (end 115.75 233.8399) (width 0.2) (layer "B.Cu") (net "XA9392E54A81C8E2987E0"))
 (segment (start 115.75 233.8399) (end 115.75 229.55) (width 0.2) (layer "B.Cu") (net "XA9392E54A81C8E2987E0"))
 (segment (start 115.6415 235.1089) (end 115.6415 240.5085) (width 0.2) (layer "F.Cu") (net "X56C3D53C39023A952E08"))
 (segment (start 115.6415 240.5085) (end 112 244.15) (width 0.2) (layer "F.Cu") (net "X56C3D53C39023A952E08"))
 (via (at 115.6415 235.1089) (size 0.6) (drill 0.3) (layers "F.Cu" "B.Cu") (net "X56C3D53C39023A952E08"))
 (segment (start 118.25 232.5004) (end 118.25 229.55) (width 0.2) (layer "B.Cu") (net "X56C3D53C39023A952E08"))
 (segment (start 115.6415 235.1089) (end 118.25 232.5004) (width 0.2) (layer "B.Cu") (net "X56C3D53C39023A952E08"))
 (segment (start 109.5 244.15) (end 110.75 242.9) (width 0.2) (layer "B.Cu") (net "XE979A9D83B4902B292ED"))
 (segment (start 110.75 242.9) (end 110.75 236.55) (width 0.2) (layer "B.Cu") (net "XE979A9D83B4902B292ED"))
 (segment (start 109.5 231.1175) (end 111.6322 233.2497) (width 0.2) (layer "F.Cu") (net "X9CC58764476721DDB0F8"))
 (segment (start 109.5 225.85) (end 109.5 231.1175) (width 0.2) (layer "F.Cu") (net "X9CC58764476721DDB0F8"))
 (via (at 111.6322 233.2497) (size 0.6) (drill 0.3) (layers "F.Cu" "B.Cu") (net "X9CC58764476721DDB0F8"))
 (segment (start 113.25 234.8675) (end 113.25 236.55) (width 0.2) (layer "B.Cu") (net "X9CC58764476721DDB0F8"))
 (segment (start 111.6322 233.2497) (end 113.25 234.8675) (width 0.2) (layer "B.Cu") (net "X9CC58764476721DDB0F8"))
 (segment (start 112 231.6786) (end 112 225.85) (width 0.2) (layer "F.Cu") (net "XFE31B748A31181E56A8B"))
 (segment (start 114.9315 234.1358) (end 114.4572 234.1358) (width 0.2) (layer "F.Cu") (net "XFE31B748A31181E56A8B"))
 (segment (start 114.4572 234.1358) (end 112 231.6786) (width 0.2) (layer "F.Cu") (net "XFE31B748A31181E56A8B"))
 (via (at 114.9315 234.1358) (size 0.6) (drill 0.3) (layers "F.Cu" "B.Cu") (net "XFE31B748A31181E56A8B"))
 (segment (start 114.9315 234.1358) (end 114.9315 235.2501) (width 0.2) (layer "B.Cu") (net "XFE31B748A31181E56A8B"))
 (segment (start 114.9315 235.2501) (end 115.75 236.0686) (width 0.2) (layer "B.Cu") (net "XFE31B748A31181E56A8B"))
 (segment (start 115.75 236.0686) (end 115.75 236.55) (width 0.2) (layer "B.Cu") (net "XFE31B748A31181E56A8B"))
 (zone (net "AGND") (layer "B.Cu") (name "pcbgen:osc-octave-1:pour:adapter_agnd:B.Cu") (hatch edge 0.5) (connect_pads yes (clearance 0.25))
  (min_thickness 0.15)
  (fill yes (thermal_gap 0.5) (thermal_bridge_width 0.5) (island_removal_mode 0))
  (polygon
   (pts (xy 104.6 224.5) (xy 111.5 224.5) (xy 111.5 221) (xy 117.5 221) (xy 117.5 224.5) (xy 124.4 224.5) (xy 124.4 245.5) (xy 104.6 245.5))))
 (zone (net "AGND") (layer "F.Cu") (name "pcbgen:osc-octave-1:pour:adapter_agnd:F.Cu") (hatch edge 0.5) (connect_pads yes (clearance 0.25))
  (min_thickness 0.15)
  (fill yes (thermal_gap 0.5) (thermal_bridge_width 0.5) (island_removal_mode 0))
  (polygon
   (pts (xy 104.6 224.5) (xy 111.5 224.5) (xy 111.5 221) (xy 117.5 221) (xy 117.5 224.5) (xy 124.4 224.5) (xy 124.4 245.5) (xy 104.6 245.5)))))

